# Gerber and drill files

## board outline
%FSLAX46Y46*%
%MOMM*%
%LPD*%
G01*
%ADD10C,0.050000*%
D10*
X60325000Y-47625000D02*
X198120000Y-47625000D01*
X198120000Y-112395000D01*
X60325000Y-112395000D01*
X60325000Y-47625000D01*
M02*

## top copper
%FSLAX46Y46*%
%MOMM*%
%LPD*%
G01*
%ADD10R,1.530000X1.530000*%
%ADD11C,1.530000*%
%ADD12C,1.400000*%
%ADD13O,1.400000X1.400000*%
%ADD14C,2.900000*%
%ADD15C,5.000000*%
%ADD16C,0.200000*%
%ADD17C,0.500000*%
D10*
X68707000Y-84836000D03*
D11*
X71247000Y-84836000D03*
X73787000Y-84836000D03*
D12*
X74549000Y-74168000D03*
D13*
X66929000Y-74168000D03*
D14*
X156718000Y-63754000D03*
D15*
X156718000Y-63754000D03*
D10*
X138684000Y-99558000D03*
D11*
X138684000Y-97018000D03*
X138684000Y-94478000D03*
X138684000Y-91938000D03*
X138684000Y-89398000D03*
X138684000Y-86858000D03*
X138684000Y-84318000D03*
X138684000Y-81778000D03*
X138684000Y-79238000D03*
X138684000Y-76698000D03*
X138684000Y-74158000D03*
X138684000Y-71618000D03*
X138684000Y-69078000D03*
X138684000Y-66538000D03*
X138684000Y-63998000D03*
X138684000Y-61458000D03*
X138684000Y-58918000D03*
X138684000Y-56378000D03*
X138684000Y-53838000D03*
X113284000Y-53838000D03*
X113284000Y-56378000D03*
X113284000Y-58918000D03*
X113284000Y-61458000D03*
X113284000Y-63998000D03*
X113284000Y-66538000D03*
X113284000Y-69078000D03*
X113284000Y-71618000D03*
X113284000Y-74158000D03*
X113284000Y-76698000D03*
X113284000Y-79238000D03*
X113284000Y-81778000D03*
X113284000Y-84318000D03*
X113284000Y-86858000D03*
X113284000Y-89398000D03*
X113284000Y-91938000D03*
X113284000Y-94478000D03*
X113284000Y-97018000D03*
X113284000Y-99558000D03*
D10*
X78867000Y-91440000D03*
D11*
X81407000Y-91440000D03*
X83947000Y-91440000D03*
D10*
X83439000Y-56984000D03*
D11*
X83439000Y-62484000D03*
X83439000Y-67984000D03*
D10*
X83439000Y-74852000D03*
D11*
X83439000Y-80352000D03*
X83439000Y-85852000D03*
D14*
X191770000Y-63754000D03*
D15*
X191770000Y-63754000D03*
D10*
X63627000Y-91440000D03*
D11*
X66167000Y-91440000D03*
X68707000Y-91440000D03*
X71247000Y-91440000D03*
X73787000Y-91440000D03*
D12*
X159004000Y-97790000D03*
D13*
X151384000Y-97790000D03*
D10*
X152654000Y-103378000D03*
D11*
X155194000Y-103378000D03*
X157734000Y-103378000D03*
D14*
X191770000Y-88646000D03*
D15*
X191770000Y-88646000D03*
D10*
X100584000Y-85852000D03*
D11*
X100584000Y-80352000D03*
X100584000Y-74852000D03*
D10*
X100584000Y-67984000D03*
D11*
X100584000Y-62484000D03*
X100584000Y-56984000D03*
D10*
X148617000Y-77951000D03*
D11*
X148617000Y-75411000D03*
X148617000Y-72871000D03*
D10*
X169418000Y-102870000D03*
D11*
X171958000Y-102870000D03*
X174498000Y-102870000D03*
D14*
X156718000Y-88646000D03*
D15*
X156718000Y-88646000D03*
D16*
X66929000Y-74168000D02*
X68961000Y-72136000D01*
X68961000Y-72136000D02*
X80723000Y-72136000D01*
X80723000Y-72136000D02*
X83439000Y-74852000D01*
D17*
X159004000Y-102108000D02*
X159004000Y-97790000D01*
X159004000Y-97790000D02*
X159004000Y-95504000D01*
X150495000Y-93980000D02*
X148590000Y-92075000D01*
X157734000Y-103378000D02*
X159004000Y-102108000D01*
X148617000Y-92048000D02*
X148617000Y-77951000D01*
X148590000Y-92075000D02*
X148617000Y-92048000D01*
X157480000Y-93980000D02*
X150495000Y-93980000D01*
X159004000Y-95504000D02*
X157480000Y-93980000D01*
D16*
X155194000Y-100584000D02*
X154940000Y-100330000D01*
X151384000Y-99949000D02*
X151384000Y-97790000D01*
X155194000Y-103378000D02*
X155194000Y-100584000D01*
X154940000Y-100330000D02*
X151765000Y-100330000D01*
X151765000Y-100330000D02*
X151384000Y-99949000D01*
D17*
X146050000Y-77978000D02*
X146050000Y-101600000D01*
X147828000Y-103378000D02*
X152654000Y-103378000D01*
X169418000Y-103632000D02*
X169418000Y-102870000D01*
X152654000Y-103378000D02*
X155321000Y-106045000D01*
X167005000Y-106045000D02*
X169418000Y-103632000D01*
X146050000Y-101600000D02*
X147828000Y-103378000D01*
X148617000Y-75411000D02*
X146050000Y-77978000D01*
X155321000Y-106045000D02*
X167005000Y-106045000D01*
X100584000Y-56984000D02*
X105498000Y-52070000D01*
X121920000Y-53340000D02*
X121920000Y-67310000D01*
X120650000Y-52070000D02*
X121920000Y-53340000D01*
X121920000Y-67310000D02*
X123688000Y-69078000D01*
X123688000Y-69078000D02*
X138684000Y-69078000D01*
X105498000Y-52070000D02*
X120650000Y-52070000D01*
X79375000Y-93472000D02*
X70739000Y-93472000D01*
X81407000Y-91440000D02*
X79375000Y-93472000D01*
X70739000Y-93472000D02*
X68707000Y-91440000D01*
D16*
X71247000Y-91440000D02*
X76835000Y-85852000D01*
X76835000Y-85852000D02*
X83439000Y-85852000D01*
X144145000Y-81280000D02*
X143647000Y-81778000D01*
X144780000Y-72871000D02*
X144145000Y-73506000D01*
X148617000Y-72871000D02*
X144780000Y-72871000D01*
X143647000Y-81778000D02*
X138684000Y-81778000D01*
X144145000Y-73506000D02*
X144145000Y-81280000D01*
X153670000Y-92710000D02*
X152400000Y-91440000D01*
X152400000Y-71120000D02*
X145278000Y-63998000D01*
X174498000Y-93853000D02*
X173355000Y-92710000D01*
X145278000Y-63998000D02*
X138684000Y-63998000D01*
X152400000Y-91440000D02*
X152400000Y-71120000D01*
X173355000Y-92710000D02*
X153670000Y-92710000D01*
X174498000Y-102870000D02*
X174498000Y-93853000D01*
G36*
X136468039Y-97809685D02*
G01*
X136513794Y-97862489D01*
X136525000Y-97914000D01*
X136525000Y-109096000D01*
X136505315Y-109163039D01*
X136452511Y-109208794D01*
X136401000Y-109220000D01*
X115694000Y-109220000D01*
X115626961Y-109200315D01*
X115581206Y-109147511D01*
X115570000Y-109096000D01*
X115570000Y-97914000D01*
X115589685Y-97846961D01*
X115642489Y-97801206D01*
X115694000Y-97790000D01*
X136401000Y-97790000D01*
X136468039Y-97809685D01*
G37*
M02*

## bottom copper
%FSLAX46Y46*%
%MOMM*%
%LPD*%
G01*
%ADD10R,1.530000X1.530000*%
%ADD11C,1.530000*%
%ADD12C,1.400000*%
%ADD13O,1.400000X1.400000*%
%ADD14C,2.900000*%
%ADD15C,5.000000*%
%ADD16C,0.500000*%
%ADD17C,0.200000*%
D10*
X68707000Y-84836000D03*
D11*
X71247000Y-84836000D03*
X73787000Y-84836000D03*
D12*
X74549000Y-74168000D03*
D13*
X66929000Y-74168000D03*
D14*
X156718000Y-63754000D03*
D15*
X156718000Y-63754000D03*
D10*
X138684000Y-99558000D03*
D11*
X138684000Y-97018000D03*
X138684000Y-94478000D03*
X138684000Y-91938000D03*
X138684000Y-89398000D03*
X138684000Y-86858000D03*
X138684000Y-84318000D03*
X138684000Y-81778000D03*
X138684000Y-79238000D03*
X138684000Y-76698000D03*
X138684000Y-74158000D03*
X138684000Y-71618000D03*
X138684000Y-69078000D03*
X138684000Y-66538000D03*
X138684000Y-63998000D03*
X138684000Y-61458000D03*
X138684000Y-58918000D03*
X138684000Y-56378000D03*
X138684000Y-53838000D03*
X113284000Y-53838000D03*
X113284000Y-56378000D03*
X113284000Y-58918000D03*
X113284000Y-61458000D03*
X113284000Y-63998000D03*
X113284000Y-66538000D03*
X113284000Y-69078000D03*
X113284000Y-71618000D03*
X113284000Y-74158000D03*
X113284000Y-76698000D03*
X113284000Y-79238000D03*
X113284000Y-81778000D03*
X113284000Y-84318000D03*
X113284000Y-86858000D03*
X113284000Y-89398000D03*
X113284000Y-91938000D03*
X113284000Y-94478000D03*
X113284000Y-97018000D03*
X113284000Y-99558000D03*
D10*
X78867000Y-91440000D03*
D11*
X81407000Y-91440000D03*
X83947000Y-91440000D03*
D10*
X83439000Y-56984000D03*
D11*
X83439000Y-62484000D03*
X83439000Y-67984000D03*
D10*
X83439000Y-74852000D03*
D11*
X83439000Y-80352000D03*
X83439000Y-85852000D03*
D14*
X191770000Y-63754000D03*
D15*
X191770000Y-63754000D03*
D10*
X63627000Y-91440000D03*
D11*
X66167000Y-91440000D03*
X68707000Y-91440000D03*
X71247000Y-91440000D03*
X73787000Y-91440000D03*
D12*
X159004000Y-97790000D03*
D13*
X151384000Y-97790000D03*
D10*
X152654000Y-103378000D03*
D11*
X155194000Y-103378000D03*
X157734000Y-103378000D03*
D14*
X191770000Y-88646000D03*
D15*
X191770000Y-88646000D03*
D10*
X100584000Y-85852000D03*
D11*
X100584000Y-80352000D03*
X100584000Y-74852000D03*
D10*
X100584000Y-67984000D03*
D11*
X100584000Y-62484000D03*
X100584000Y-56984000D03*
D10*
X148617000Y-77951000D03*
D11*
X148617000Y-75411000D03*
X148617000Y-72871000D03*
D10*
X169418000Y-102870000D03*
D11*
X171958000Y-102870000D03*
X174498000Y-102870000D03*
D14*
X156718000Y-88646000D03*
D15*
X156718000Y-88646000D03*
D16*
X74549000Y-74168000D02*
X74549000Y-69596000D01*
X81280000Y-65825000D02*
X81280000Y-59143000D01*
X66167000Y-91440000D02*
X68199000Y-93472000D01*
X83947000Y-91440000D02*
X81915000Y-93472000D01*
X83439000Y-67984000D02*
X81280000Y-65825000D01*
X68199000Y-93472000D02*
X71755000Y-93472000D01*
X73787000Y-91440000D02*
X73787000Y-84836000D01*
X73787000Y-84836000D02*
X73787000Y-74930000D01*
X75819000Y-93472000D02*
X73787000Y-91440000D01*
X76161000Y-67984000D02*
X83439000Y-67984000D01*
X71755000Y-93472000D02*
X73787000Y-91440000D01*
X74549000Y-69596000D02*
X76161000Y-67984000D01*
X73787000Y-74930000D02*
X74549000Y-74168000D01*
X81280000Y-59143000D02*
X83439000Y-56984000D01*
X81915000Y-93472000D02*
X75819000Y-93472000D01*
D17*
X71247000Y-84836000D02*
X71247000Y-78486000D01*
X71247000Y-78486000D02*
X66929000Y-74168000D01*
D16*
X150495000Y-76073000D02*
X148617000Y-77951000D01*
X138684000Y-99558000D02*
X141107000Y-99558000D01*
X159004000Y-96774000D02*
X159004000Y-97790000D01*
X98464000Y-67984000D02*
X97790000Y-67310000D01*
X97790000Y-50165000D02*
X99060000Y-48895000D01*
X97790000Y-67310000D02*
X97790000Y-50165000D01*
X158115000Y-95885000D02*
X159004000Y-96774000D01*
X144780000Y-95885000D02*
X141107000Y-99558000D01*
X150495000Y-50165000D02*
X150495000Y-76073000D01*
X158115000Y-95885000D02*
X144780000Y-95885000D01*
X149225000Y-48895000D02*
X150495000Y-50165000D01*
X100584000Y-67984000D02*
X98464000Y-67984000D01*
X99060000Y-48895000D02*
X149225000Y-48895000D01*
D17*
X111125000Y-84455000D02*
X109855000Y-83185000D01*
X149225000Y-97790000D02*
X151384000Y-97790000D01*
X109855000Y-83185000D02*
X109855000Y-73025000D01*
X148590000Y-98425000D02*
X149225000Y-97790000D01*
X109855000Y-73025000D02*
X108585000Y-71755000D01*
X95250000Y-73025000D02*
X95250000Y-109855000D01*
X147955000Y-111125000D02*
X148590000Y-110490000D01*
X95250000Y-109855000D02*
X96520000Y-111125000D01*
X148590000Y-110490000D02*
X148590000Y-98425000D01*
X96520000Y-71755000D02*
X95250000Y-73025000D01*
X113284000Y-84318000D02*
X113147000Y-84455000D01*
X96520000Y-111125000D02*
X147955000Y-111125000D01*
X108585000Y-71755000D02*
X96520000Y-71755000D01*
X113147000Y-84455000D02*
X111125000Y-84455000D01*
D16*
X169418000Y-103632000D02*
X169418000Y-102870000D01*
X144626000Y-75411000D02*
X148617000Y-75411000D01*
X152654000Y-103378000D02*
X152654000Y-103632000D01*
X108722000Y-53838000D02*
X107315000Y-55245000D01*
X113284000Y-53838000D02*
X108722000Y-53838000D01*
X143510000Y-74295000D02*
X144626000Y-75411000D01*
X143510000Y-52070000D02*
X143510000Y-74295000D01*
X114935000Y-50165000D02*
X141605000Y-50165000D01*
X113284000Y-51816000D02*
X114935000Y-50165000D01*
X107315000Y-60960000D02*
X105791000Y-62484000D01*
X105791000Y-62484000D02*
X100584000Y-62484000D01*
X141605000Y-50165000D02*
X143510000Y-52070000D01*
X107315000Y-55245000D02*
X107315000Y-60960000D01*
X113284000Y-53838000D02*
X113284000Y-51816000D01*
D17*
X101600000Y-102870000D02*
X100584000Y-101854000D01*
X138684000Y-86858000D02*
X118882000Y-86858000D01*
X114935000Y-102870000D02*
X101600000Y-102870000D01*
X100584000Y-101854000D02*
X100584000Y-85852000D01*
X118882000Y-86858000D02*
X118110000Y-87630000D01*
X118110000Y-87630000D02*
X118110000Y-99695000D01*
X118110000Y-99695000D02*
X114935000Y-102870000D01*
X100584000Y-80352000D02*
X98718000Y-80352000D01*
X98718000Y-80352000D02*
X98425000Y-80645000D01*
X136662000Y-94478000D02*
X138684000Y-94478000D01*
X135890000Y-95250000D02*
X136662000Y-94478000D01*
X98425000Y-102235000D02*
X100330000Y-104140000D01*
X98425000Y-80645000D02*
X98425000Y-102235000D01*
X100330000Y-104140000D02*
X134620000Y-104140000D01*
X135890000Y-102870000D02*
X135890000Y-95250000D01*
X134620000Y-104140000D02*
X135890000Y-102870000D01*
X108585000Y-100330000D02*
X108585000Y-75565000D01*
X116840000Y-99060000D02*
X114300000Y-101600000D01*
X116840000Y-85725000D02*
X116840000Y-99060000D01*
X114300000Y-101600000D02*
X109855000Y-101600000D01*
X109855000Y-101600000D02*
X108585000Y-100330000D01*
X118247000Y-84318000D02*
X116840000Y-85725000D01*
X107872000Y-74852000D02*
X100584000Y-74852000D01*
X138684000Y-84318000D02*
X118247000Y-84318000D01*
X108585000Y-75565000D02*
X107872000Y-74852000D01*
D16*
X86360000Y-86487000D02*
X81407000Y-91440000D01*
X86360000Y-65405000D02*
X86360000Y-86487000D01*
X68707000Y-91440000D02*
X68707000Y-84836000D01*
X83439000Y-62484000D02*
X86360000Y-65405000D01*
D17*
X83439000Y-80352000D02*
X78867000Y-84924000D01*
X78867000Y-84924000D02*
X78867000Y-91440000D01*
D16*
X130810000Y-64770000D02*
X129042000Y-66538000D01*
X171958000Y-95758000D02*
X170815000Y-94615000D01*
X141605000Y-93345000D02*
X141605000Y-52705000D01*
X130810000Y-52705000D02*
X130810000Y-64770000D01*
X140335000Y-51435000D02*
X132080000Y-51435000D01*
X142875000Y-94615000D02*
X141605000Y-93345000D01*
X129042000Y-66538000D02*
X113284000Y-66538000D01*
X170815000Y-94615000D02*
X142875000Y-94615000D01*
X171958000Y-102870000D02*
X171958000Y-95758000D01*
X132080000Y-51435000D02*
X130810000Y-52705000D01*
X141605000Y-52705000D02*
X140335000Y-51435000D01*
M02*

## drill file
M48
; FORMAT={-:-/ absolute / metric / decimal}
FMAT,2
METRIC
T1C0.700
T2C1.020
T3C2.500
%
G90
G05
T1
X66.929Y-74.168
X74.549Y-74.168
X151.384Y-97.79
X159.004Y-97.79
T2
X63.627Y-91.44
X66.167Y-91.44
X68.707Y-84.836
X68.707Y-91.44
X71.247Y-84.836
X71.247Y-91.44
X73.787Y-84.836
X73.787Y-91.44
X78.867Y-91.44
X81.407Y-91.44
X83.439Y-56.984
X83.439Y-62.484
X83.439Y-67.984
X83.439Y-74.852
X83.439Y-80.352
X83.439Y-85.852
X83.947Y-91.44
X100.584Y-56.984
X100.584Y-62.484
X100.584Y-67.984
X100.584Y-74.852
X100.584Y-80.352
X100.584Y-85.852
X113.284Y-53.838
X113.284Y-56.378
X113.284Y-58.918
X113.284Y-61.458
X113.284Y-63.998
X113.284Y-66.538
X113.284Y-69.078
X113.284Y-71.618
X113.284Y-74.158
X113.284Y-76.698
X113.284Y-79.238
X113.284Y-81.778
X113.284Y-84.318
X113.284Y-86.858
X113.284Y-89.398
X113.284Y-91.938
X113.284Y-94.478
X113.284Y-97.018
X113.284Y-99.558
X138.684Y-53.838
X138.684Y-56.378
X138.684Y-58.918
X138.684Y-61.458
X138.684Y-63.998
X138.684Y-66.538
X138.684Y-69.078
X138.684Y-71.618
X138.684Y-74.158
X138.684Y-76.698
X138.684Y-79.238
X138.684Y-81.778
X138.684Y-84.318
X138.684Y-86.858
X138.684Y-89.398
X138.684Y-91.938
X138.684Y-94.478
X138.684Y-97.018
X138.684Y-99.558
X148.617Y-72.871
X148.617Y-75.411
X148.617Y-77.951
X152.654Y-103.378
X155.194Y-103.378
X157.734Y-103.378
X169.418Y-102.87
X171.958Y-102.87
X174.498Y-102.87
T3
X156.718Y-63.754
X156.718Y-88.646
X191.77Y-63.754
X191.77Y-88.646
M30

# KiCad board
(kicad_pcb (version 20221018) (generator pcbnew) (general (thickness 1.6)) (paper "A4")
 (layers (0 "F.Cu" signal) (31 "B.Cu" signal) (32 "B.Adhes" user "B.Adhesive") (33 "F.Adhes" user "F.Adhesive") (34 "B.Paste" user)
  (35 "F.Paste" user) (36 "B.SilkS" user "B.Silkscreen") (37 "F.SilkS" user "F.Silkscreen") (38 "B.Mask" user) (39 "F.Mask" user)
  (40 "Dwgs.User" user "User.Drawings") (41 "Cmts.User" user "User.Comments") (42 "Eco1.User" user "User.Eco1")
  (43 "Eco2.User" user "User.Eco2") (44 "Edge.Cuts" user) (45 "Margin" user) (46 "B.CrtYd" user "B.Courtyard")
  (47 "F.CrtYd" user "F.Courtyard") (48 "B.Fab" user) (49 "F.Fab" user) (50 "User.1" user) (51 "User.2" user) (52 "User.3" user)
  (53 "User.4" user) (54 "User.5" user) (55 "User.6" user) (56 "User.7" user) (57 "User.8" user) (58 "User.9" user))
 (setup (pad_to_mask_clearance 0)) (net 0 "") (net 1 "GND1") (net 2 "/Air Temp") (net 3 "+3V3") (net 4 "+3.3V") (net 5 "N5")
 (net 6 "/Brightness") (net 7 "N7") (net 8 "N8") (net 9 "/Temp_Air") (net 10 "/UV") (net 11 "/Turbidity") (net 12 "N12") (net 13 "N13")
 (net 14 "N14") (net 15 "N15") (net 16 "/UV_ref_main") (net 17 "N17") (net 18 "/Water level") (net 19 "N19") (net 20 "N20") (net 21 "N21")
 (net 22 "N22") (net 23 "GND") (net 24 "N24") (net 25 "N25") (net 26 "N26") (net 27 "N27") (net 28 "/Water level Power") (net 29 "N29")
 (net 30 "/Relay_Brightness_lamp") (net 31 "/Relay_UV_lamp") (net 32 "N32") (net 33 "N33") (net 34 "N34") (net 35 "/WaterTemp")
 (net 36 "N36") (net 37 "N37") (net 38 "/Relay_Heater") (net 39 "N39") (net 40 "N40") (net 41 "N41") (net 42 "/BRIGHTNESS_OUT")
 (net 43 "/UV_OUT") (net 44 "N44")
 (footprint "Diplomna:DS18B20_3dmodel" (layer "F.Cu") (at 76.327 87.376)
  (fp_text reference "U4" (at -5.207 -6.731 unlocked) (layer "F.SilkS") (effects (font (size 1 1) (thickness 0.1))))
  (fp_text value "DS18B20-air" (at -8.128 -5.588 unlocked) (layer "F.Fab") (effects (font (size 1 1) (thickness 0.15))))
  (pad "1" thru_hole rect (at -7.62 -2.54) (size 1.53 1.53) (drill 1.02) (layers "*.Cu" "*.Mask") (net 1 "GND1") (solder_mask_margin 0.102))
  (pad "2" thru_hole circle (at -5.08 -2.54) (size 1.53 1.53) (drill 1.02) (layers "*.Cu" "*.Mask") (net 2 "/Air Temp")
   (solder_mask_margin 0.102))
  (pad "3" thru_hole circle (at -2.54 -2.54) (size 1.53 1.53) (drill 1.02) (layers "*.Cu" "*.Mask") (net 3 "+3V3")
   (solder_mask_margin 0.102)))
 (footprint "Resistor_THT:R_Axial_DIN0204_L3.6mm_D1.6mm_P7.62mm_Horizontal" (layer "F.Cu") (at 74.549 74.168 180)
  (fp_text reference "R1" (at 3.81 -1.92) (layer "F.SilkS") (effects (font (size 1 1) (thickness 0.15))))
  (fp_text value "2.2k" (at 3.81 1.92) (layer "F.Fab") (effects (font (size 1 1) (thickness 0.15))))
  (pad "1" thru_hole circle (at 0 0 180) (size 1.4 1.4) (drill 0.7) (layers "*.Cu" "*.Mask") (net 3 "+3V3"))
  (pad "2" thru_hole oval (at 7.62 0 180) (size 1.4 1.4) (drill 0.7) (layers "*.Cu" "*.Mask") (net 2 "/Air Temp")))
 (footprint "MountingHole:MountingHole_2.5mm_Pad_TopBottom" (layer "F.Cu") (at 156.718 63.754)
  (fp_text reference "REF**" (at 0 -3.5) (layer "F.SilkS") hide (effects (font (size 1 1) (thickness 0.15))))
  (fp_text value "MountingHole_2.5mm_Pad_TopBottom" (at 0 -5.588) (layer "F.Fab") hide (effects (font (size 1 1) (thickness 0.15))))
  (pad "1" thru_hole circle (at 0 0) (size 2.9 2.9) (drill 2.5) (layers "*.Cu" "*.Mask"))
  (pad "1" connect circle (at 0 0) (size 5 5) (layers "F.Cu" "F.Mask"))
  (pad "1" connect circle (at 0 0) (size 5 5) (layers "B.Cu" "B.Mask")))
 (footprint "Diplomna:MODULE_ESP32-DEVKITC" (layer "F.Cu") (at 125.984 76.708 180)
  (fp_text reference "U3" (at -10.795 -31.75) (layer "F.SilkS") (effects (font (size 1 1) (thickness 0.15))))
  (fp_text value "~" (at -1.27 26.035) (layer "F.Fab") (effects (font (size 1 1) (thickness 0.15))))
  (pad "1" thru_hole rect (at -12.7 -22.85 180) (size 1.53 1.53) (drill 1.02) (layers "*.Cu" "*.Mask") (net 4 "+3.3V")
   (solder_mask_margin 0.102))
  (pad "2" thru_hole circle (at -12.7 -20.31 180) (size 1.53 1.53) (drill 1.02) (layers "*.Cu" "*.Mask") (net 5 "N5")
   (solder_mask_margin 0.102))
  (pad "3" thru_hole circle (at -12.7 -17.77 180) (size 1.53 1.53) (drill 1.02) (layers "*.Cu" "*.Mask") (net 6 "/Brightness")
   (solder_mask_margin 0.102))
  (pad "4" thru_hole circle (at -12.7 -15.23 180) (size 1.53 1.53) (drill 1.02) (layers "*.Cu" "*.Mask") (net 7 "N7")
   (solder_mask_margin 0.102))
  (pad "5" thru_hole circle (at -12.7 -12.69 180) (size 1.53 1.53) (drill 1.02) (layers "*.Cu" "*.Mask") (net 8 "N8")
   (solder_mask_margin 0.102))
  (pad "6" thru_hole circle (at -12.7 -10.15 180) (size 1.53 1.53) (drill 1.02) (layers "*.Cu" "*.Mask") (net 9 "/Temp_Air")
   (solder_mask_margin 0.102))
  (pad "7" thru_hole circle (at -12.7 -7.61 180) (size 1.53 1.53) (drill 1.02) (layers "*.Cu" "*.Mask") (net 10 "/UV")
   (solder_mask_margin 0.102))
  (pad "8" thru_hole circle (at -12.7 -5.07 180) (size 1.53 1.53) (drill 1.02) (layers "*.Cu" "*.Mask") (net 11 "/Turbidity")
   (solder_mask_margin 0.102))
  (pad "9" thru_hole circle (at -12.7 -2.53 180) (size 1.53 1.53) (drill 1.02) (layers "*.Cu" "*.Mask") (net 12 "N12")
   (solder_mask_margin 0.102))
  (pad "10" thru_hole circle (at -12.7 0.01 180) (size 1.53 1.53) (drill 1.02) (layers "*.Cu" "*.Mask") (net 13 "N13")
   (solder_mask_margin 0.102))
  (pad "11" thru_hole circle (at -12.7 2.55 180) (size 1.53 1.53) (drill 1.02) (layers "*.Cu" "*.Mask") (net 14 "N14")
   (solder_mask_margin 0.102))
  (pad "12" thru_hole circle (at -12.7 5.09 180) (size 1.53 1.53) (drill 1.02) (layers "*.Cu" "*.Mask") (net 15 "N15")
   (solder_mask_margin 0.102))
  (pad "13" thru_hole circle (at -12.7 7.63 180) (size 1.53 1.53) (drill 1.02) (layers "*.Cu" "*.Mask") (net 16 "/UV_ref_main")
   (solder_mask_margin 0.102))
  (pad "14" thru_hole circle (at -12.7 10.17 180) (size 1.53 1.53) (drill 1.02) (layers "*.Cu" "*.Mask") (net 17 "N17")
   (solder_mask_margin 0.102))
  (pad "15" thru_hole circle (at -12.7 12.71 180) (size 1.53 1.53) (drill 1.02) (layers "*.Cu" "*.Mask") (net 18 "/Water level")
   (solder_mask_margin 0.102))
  (pad "16" thru_hole circle (at -12.7 15.25 180) (size 1.53 1.53) (drill 1.02) (layers "*.Cu" "*.Mask") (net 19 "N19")
   (solder_mask_margin 0.102))
  (pad "17" thru_hole circle (at -12.7 17.79 180) (size 1.53 1.53) (drill 1.02) (layers "*.Cu" "*.Mask") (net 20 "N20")
   (solder_mask_margin 0.102))
  (pad "18" thru_hole circle (at -12.7 20.33 180) (size 1.53 1.53) (drill 1.02) (layers "*.Cu" "*.Mask") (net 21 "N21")
   (solder_mask_margin 0.102))
  (pad "19" thru_hole circle (at -12.7 22.87 180) (size 1.53 1.53) (drill 1.02) (layers "*.Cu" "*.Mask") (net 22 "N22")
   (solder_mask_margin 0.102))
  (pad "20" thru_hole circle (at 12.7 22.87 180) (size 1.53 1.53) (drill 1.02) (layers "*.Cu" "*.Mask") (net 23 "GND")
   (solder_mask_margin 0.102))
  (pad "21" thru_hole circle (at 12.7 20.33 180) (size 1.53 1.53) (drill 1.02) (layers "*.Cu" "*.Mask") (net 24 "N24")
   (solder_mask_margin 0.102))
  (pad "22" thru_hole circle (at 12.7 17.79 180) (size 1.53 1.53) (drill 1.02) (layers "*.Cu" "*.Mask") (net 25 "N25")
   (solder_mask_margin 0.102))
  (pad "23" thru_hole circle (at 12.7 15.25 180) (size 1.53 1.53) (drill 1.02) (layers "*.Cu" "*.Mask") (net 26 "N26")
   (solder_mask_margin 0.102))
  (pad "24" thru_hole circle (at 12.7 12.71 180) (size 1.53 1.53) (drill 1.02) (layers "*.Cu" "*.Mask") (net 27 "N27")
   (solder_mask_margin 0.102))
  (pad "25" thru_hole circle (at 12.7 10.17 180) (size 1.53 1.53) (drill 1.02) (layers "*.Cu" "*.Mask") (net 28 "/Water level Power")
   (solder_mask_margin 0.102))
  (pad "26" thru_hole circle (at 12.7 7.63 180) (size 1.53 1.53) (drill 1.02) (layers "*.Cu" "*.Mask") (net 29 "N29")
   (solder_mask_margin 0.102))
  (pad "27" thru_hole circle (at 12.7 5.09 180) (size 1.53 1.53) (drill 1.02) (layers "*.Cu" "*.Mask") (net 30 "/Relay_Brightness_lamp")
   (solder_mask_margin 0.102))
  (pad "28" thru_hole circle (at 12.7 2.55 180) (size 1.53 1.53) (drill 1.02) (layers "*.Cu" "*.Mask") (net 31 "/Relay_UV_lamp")
   (solder_mask_margin 0.102))
  (pad "29" thru_hole circle (at 12.7 0.01 180) (size 1.53 1.53) (drill 1.02) (layers "*.Cu" "*.Mask") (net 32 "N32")
   (solder_mask_margin 0.102))
  (pad "30" thru_hole circle (at 12.7 -2.53 180) (size 1.53 1.53) (drill 1.02) (layers "*.Cu" "*.Mask") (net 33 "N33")
   (solder_mask_margin 0.102))
  (pad "31" thru_hole circle (at 12.7 -5.07 180) (size 1.53 1.53) (drill 1.02) (layers "*.Cu" "*.Mask") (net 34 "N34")
   (solder_mask_margin 0.102))
  (pad "32" thru_hole circle (at 12.7 -7.61 180) (size 1.53 1.53) (drill 1.02) (layers "*.Cu" "*.Mask") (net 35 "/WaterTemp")
   (solder_mask_margin 0.102))
  (pad "33" thru_hole circle (at 12.7 -10.15 180) (size 1.53 1.53) (drill 1.02) (layers "*.Cu" "*.Mask") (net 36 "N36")
   (solder_mask_margin 0.102))
  (pad "34" thru_hole circle (at 12.7 -12.69 180) (size 1.53 1.53) (drill 1.02) (layers "*.Cu" "*.Mask") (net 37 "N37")
   (solder_mask_margin 0.102))
  (pad "35" thru_hole circle (at 12.7 -15.23 180) (size 1.53 1.53) (drill 1.02) (layers "*.Cu" "*.Mask") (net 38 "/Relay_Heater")
   (solder_mask_margin 0.102))
  (pad "36" thru_hole circle (at 12.7 -17.77 180) (size 1.53 1.53) (drill 1.02) (layers "*.Cu" "*.Mask") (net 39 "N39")
   (solder_mask_margin 0.102))
  (pad "37" thru_hole circle (at 12.7 -20.31 180) (size 1.53 1.53) (drill 1.02) (layers "*.Cu" "*.Mask") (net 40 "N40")
   (solder_mask_margin 0.102))
  (pad "38" thru_hole circle (at 12.7 -22.85 180) (size 1.53 1.53) (drill 1.02) (layers "*.Cu" "*.Mask") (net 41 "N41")
   (solder_mask_margin 0.102)))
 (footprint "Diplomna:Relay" (layer "F.Cu") (at 254.508 101.092 -90)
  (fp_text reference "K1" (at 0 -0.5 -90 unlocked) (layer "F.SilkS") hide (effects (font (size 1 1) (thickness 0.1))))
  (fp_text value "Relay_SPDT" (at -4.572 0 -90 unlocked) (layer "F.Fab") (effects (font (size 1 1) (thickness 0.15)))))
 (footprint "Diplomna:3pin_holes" (layer "F.Cu") (at 86.487 93.98)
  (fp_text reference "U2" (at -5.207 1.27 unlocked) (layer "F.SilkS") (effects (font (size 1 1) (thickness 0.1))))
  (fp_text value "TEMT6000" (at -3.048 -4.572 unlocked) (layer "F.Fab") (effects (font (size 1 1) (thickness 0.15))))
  (pad "1" thru_hole rect (at -7.62 -2.54) (size 1.53 1.53) (drill 1.02) (layers "*.Cu" "*.Mask") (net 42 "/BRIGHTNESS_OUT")
   (solder_mask_margin 0.102))
  (pad "2" thru_hole circle (at -5.08 -2.54) (size 1.53 1.53) (drill 1.02) (layers "*.Cu" "*.Mask") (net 1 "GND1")
   (solder_mask_margin 0.102))
  (pad "3" thru_hole circle (at -2.54 -2.54) (size 1.53 1.53) (drill 1.02) (layers "*.Cu" "*.Mask") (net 3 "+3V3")
   (solder_mask_margin 0.102)))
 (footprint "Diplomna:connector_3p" (layer "F.Cu") (at 83.439 62.484 -90)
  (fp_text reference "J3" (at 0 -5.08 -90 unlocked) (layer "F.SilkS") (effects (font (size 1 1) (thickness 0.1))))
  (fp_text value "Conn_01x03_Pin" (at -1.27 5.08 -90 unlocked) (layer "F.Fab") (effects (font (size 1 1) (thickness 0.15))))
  (pad "1" thru_hole rect (at -5.5 0 270) (size 1.53 1.53) (drill 1.02) (layers "*.Cu" "*.Mask") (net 3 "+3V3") (solder_mask_margin 0.102))
  (pad "2" thru_hole circle (at 0 0 270) (size 1.53 1.53) (drill 1.02) (layers "*.Cu" "*.Mask") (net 1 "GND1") (solder_mask_margin 0.102))
  (pad "3" thru_hole circle (at 5.5 0 270) (size 1.53 1.53) (drill 1.02) (layers "*.Cu" "*.Mask") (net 3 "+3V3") (solder_mask_margin 0.102)))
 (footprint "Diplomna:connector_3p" (layer "F.Cu") (at 83.439 80.352 -90)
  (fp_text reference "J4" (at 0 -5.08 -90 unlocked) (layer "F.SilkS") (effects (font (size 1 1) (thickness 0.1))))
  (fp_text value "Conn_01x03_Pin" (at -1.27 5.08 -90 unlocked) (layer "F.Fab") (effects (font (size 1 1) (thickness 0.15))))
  (pad "1" thru_hole rect (at -5.5 0 270) (size 1.53 1.53) (drill 1.02) (layers "*.Cu" "*.Mask") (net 2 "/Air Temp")
   (solder_mask_margin 0.102))
  (pad "2" thru_hole circle (at 0 0 270) (size 1.53 1.53) (drill 1.02) (layers "*.Cu" "*.Mask") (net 42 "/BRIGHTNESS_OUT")
   (solder_mask_margin 0.102))
  (pad "3" thru_hole circle (at 5.5 0 270) (size 1.53 1.53) (drill 1.02) (layers "*.Cu" "*.Mask") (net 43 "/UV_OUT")
   (solder_mask_margin 0.102)))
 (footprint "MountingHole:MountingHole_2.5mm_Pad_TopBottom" (layer "F.Cu") (at 191.77 63.754)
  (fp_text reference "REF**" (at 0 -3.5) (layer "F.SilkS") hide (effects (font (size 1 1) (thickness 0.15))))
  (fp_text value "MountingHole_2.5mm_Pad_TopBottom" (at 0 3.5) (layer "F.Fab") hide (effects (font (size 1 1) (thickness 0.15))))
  (pad "1" thru_hole circle (at 0 0) (size 2.9 2.9) (drill 2.5) (layers "*.Cu" "*.Mask"))
  (pad "1" connect circle (at 0 0) (size 5 5) (layers "F.Cu" "F.Mask"))
  (pad "1" connect circle (at 0 0) (size 5 5) (layers "B.Cu" "B.Mask")))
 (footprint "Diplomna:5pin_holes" (layer "F.Cu") (at 78.867 97.155)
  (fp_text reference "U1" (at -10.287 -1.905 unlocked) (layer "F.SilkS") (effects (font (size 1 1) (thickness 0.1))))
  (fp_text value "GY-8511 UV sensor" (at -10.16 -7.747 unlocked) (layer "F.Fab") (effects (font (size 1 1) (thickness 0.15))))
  (pad "1" thru_hole rect (at -15.24 -5.715) (size 1.53 1.53) (drill 1.02) (layers "*.Cu" "*.Mask") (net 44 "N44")
   (solder_mask_margin 0.102))
  (pad "2" thru_hole circle (at -12.7 -5.715) (size 1.53 1.53) (drill 1.02) (layers "*.Cu" "*.Mask") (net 3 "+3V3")
   (solder_mask_margin 0.102))
  (pad "3" thru_hole circle (at -10.16 -5.715) (size 1.53 1.53) (drill 1.02) (layers "*.Cu" "*.Mask") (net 1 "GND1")
   (solder_mask_margin 0.102))
  (pad "4" thru_hole circle (at -7.62 -5.715) (size 1.53 1.53) (drill 1.02) (layers "*.Cu" "*.Mask") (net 43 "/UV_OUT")
   (solder_mask_margin 0.102))
  (pad "5" thru_hole circle (at -5.08 -5.715) (size 1.53 1.53) (drill 1.02) (layers "*.Cu" "*.Mask") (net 3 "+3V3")
   (solder_mask_margin 0.102)))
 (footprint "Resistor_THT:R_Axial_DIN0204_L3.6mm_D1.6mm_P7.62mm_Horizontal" (layer "F.Cu") (at 159.004 97.79 180)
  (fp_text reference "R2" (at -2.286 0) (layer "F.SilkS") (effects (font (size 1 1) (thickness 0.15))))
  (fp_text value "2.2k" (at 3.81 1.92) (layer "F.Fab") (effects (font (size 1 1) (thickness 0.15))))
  (pad "1" thru_hole circle (at 0 0 180) (size 1.4 1.4) (drill 0.7) (layers "*.Cu" "*.Mask") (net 4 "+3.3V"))
  (pad "2" thru_hole oval (at 7.62 0 180) (size 1.4 1.4) (drill 0.7) (layers "*.Cu" "*.Mask") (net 35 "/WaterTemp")))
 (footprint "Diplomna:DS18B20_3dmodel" (layer "F.Cu") (at 160.274 105.918)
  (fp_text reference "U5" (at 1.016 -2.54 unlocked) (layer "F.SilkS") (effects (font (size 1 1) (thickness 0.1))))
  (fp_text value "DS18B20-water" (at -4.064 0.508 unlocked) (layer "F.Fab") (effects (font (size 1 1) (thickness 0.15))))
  (pad "1" thru_hole rect (at -7.62 -2.54) (size 1.53 1.53) (drill 1.02) (layers "*.Cu" "*.Mask") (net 23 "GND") (solder_mask_margin 0.102))
  (pad "2" thru_hole circle (at -5.08 -2.54) (size 1.53 1.53) (drill 1.02) (layers "*.Cu" "*.Mask") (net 35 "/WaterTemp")
   (solder_mask_margin 0.102))
  (pad "3" thru_hole circle (at -2.54 -2.54) (size 1.53 1.53) (drill 1.02) (layers "*.Cu" "*.Mask") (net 4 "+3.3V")
   (solder_mask_margin 0.102)))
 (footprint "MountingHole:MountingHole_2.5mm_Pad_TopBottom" (layer "F.Cu") (at 191.77 88.646)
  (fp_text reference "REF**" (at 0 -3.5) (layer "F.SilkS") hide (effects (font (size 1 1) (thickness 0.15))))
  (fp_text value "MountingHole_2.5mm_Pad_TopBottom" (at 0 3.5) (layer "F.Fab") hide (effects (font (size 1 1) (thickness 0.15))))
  (pad "1" thru_hole circle (at 0 0) (size 2.9 2.9) (drill 2.5) (layers "*.Cu" "*.Mask"))
  (pad "1" connect circle (at 0 0) (size 5 5) (layers "F.Cu" "F.Mask"))
  (pad "1" connect circle (at 0 0) (size 5 5) (layers "B.Cu" "B.Mask")))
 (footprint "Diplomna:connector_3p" (layer "F.Cu") (at 100.584 80.352 90)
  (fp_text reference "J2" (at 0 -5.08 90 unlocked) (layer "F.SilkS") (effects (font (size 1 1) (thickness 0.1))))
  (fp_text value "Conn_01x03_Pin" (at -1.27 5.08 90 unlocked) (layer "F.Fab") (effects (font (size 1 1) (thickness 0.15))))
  (pad "1" thru_hole rect (at -5.5 0 90) (size 1.53 1.53) (drill 1.02) (layers "*.Cu" "*.Mask") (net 9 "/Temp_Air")
   (solder_mask_margin 0.102))
  (pad "2" thru_hole circle (at 0 0 90) (size 1.53 1.53) (drill 1.02) (layers "*.Cu" "*.Mask") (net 6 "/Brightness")
   (solder_mask_margin 0.102))
  (pad "3" thru_hole circle (at 5.5 0 90) (size 1.53 1.53) (drill 1.02) (layers "*.Cu" "*.Mask") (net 10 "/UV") (solder_mask_margin 0.102)))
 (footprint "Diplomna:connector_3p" (layer "F.Cu") (at 100.584 62.484 90)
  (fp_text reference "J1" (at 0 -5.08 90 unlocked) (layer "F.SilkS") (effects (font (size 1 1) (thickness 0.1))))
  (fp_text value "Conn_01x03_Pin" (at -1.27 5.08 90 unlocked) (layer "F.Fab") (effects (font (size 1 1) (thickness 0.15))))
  (pad "1" thru_hole rect (at -5.5 0 90) (size 1.53 1.53) (drill 1.02) (layers "*.Cu" "*.Mask") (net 4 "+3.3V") (solder_mask_margin 0.102))
  (pad "2" thru_hole circle (at 0 0 90) (size 1.53 1.53) (drill 1.02) (layers "*.Cu" "*.Mask") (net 23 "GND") (solder_mask_margin 0.102))
  (pad "3" thru_hole circle (at 5.5 0 90) (size 1.53 1.53) (drill 1.02) (layers "*.Cu" "*.Mask") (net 16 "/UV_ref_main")
   (solder_mask_margin 0.102)))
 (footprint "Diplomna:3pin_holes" (layer "F.Cu") (at 151.157 70.331 90)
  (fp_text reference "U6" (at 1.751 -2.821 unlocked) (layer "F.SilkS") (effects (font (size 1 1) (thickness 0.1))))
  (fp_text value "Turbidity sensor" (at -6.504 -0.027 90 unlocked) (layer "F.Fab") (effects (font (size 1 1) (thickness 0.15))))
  (pad "1" thru_hole rect (at -7.62 -2.54 90) (size 1.53 1.53) (drill 1.02) (layers "*.Cu" "*.Mask") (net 4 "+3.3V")
   (solder_mask_margin 0.102))
  (pad "2" thru_hole circle (at -5.08 -2.54 90) (size 1.53 1.53) (drill 1.02) (layers "*.Cu" "*.Mask") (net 23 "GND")
   (solder_mask_margin 0.102))
  (pad "3" thru_hole circle (at -2.54 -2.54 90) (size 1.53 1.53) (drill 1.02) (layers "*.Cu" "*.Mask") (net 11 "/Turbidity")
   (solder_mask_margin 0.102)))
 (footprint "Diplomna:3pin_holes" (layer "F.Cu") (at 177.038 105.41)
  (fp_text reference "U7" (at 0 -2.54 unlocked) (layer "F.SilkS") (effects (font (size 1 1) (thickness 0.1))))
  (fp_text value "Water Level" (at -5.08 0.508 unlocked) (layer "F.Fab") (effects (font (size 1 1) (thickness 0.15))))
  (pad "1" thru_hole rect (at -7.62 -2.54) (size 1.53 1.53) (drill 1.02) (layers "*.Cu" "*.Mask") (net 23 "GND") (solder_mask_margin 0.102))
  (pad "2" thru_hole circle (at -5.08 -2.54) (size 1.53 1.53) (drill 1.02) (layers "*.Cu" "*.Mask") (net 28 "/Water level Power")
   (solder_mask_margin 0.102))
  (pad "3" thru_hole circle (at -2.54 -2.54) (size 1.53 1.53) (drill 1.02) (layers "*.Cu" "*.Mask") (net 18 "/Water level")
   (solder_mask_margin 0.102)))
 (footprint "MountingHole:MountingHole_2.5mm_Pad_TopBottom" (layer "F.Cu") (at 156.718 88.646)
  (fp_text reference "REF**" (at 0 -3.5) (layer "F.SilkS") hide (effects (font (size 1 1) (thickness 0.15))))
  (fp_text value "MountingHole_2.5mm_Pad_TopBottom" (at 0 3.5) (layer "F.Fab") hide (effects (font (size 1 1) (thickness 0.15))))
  (pad "1" thru_hole circle (at 0 0) (size 2.9 2.9) (drill 2.5) (layers "*.Cu" "*.Mask"))
  (pad "1" connect circle (at 0 0) (size 5 5) (layers "F.Cu" "F.Mask"))
  (pad "1" connect circle (at 0 0) (size 5 5) (layers "B.Cu" "B.Mask")))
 (gr_rect (start 60.325 47.625) (end 198.12 112.395) (stroke (width 0.05) (type default)) (fill none) (layer "Edge.Cuts"))
 (segment (start 74.549 74.168) (end 74.549 69.596) (width 0.5) (layer "B.Cu") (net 3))
 (segment (start 81.28 65.825) (end 81.28 59.143) (width 0.5) (layer "B.Cu") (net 3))
 (segment (start 66.167 91.44) (end 68.199 93.472) (width 0.5) (layer "B.Cu") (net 3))
 (segment (start 83.947 91.44) (end 81.915 93.472) (width 0.5) (layer "B.Cu") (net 3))
 (segment (start 83.439 67.984) (end 81.28 65.825) (width 0.5) (layer "B.Cu") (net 3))
 (segment (start 68.199 93.472) (end 71.755 93.472) (width 0.5) (layer "B.Cu") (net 3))
 (segment (start 73.787 91.44) (end 73.787 84.836) (width 0.5) (layer "B.Cu") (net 3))
 (segment (start 73.787 84.836) (end 73.787 74.93) (width 0.5) (layer "B.Cu") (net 3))
 (segment (start 75.819 93.472) (end 73.787 91.44) (width 0.5) (layer "B.Cu") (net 3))
 (segment (start 76.161 67.984) (end 83.439 67.984) (width 0.5) (layer "B.Cu") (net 3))
 (segment (start 71.755 93.472) (end 73.787 91.44) (width 0.5) (layer "B.Cu") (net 3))
 (segment (start 74.549 69.596) (end 76.161 67.984) (width 0.5) (layer "B.Cu") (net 3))
 (segment (start 73.787 74.93) (end 74.549 74.168) (width 0.5) (layer "B.Cu") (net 3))
 (segment (start 81.28 59.143) (end 83.439 56.984) (width 0.5) (layer "B.Cu") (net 3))
 (segment (start 81.915 93.472) (end 75.819 93.472) (width 0.5) (layer "B.Cu") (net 3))
 (segment (start 66.929 74.168) (end 68.961 72.136) (width 0.2) (layer "F.Cu") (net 2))
 (segment (start 68.961 72.136) (end 80.723 72.136) (width 0.2) (layer "F.Cu") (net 2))
 (segment (start 80.723 72.136) (end 83.439 74.852) (width 0.2) (layer "F.Cu") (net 2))
 (segment (start 71.247 84.836) (end 71.247 78.486) (width 0.2) (layer "B.Cu") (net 2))
 (segment (start 71.247 78.486) (end 66.929 74.168) (width 0.2) (layer "B.Cu") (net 2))
 (segment (start 159.004 102.108) (end 159.004 97.79) (width 0.5) (layer "F.Cu") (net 4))
 (segment (start 159.004 97.79) (end 159.004 95.504) (width 0.5) (layer "F.Cu") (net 4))
 (segment (start 150.495 93.98) (end 148.59 92.075) (width 0.5) (layer "F.Cu") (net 4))
 (segment (start 157.734 103.378) (end 159.004 102.108) (width 0.5) (layer "F.Cu") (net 4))
 (segment (start 148.617 92.048) (end 148.617 77.951) (width 0.5) (layer "F.Cu") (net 4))
 (segment (start 148.59 92.075) (end 148.617 92.048) (width 0.5) (layer "F.Cu") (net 4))
 (segment (start 157.48 93.98) (end 150.495 93.98) (width 0.5) (layer "F.Cu") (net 4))
 (segment (start 159.004 95.504) (end 157.48 93.98) (width 0.5) (layer "F.Cu") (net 4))
 (segment (start 150.495 76.073) (end 148.617 77.951) (width 0.5) (layer "B.Cu") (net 4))
 (segment (start 138.684 99.558) (end 141.107 99.558) (width 0.5) (layer "B.Cu") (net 4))
 (segment (start 159.004 96.774) (end 159.004 97.79) (width 0.5) (layer "B.Cu") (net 4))
 (segment (start 98.464 67.984) (end 97.79 67.31) (width 0.5) (layer "B.Cu") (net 4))
 (segment (start 97.79 50.165) (end 99.06 48.895) (width 0.5) (layer "B.Cu") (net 4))
 (segment (start 97.79 67.31) (end 97.79 50.165) (width 0.5) (layer "B.Cu") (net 4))
 (segment (start 158.115 95.885) (end 159.004 96.774) (width 0.5) (layer "B.Cu") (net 4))
 (segment (start 144.78 95.885) (end 141.107 99.558) (width 0.5) (layer "B.Cu") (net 4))
 (segment (start 150.495 50.165) (end 150.495 76.073) (width 0.5) (layer "B.Cu") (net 4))
 (segment (start 158.115 95.885) (end 144.78 95.885) (width 0.5) (layer "B.Cu") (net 4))
 (segment (start 149.225 48.895) (end 150.495 50.165) (width 0.5) (layer "B.Cu") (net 4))
 (segment (start 100.584 67.984) (end 98.464 67.984) (width 0.5) (layer "B.Cu") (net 4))
 (segment (start 99.06 48.895) (end 149.225 48.895) (width 0.5) (layer "B.Cu") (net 4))
 (segment (start 155.194 100.584) (end 154.94 100.33) (width 0.2) (layer "F.Cu") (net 35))
 (segment (start 151.384 99.949) (end 151.384 97.79) (width 0.2) (layer "F.Cu") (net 35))
 (segment (start 155.194 103.378) (end 155.194 100.584) (width 0.2) (layer "F.Cu") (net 35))
 (segment (start 154.94 100.33) (end 151.765 100.33) (width 0.2) (layer "F.Cu") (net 35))
 (segment (start 151.765 100.33) (end 151.384 99.949) (width 0.2) (layer "F.Cu") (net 35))
 (segment (start 111.125 84.455) (end 109.855 83.185) (width 0.2) (layer "B.Cu") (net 35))
 (segment (start 149.225 97.79) (end 151.384 97.79) (width 0.2) (layer "B.Cu") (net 35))
 (segment (start 109.855 83.185) (end 109.855 73.025) (width 0.2) (layer "B.Cu") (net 35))
 (segment (start 148.59 98.425) (end 149.225 97.79) (width 0.2) (layer "B.Cu") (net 35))
 (segment (start 109.855 73.025) (end 108.585 71.755) (width 0.2) (layer "B.Cu") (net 35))
 (segment (start 95.25 73.025) (end 95.25 109.855) (width 0.2) (layer "B.Cu") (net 35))
 (segment (start 147.955 111.125) (end 148.59 110.49) (width 0.2) (layer "B.Cu") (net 35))
 (segment (start 95.25 109.855) (end 96.52 111.125) (width 0.2) (layer "B.Cu") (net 35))
 (segment (start 148.59 110.49) (end 148.59 98.425) (width 0.2) (layer "B.Cu") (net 35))
 (segment (start 96.52 71.755) (end 95.25 73.025) (width 0.2) (layer "B.Cu") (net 35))
 (segment (start 113.284 84.318) (end 113.147 84.455) (width 0.2) (layer "B.Cu") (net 35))
 (segment (start 96.52 111.125) (end 147.955 111.125) (width 0.2) (layer "B.Cu") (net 35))
 (segment (start 108.585 71.755) (end 96.52 71.755) (width 0.2) (layer "B.Cu") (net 35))
 (segment (start 113.147 84.455) (end 111.125 84.455) (width 0.2) (layer "B.Cu") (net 35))
 (segment (start 146.05 77.978) (end 146.05 101.6) (width 0.5) (layer "F.Cu") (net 23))
 (segment (start 147.828 103.378) (end 152.654 103.378) (width 0.5) (layer "F.Cu") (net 23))
 (segment (start 169.418 103.632) (end 169.418 102.87) (width 0.5) (layer "F.Cu") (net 23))
 (segment (start 152.654 103.378) (end 155.321 106.045) (width 0.5) (layer "F.Cu") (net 23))
 (segment (start 167.005 106.045) (end 169.418 103.632) (width 0.5) (layer "F.Cu") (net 23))
 (segment (start 146.05 101.6) (end 147.828 103.378) (width 0.5) (layer "F.Cu") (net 23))
 (segment (start 148.617 75.411) (end 146.05 77.978) (width 0.5) (layer "F.Cu") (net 23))
 (segment (start 155.321 106.045) (end 167.005 106.045) (width 0.5) (layer "F.Cu") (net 23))
 (segment (start 169.418 103.632) (end 169.418 102.87) (width 0.5) (layer "B.Cu") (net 23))
 (segment (start 144.626 75.411) (end 148.617 75.411) (width 0.5) (layer "B.Cu") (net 23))
 (segment (start 152.654 103.378) (end 152.654 103.632) (width 0.5) (layer "B.Cu") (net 23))
 (segment (start 108.722 53.838) (end 107.315 55.245) (width 0.5) (layer "B.Cu") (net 23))
 (segment (start 113.284 53.838) (end 108.722 53.838) (width 0.5) (layer "B.Cu") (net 23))
 (segment (start 143.51 74.295) (end 144.626 75.411) (width 0.5) (layer "B.Cu") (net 23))
 (segment (start 143.51 52.07) (end 143.51 74.295) (width 0.5) (layer "B.Cu") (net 23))
 (segment (start 114.935 50.165) (end 141.605 50.165) (width 0.5) (layer "B.Cu") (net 23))
 (segment (start 113.284 51.816) (end 114.935 50.165) (width 0.5) (layer "B.Cu") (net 23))
 (segment (start 107.315 60.96) (end 105.791 62.484) (width 0.5) (layer "B.Cu") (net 23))
 (segment (start 105.791 62.484) (end 100.584 62.484) (width 0.5) (layer "B.Cu") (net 23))
 (segment (start 141.605 50.165) (end 143.51 52.07) (width 0.5) (layer "B.Cu") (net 23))
 (segment (start 107.315 55.245) (end 107.315 60.96) (width 0.5) (layer "B.Cu") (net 23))
 (segment (start 113.284 53.838) (end 113.284 51.816) (width 0.5) (layer "B.Cu") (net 23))
 (segment (start 100.584 56.984) (end 105.498 52.07) (width 0.5) (layer "F.Cu") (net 16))
 (segment (start 121.92 53.34) (end 121.92 67.31) (width 0.5) (layer "F.Cu") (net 16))
 (segment (start 120.65 52.07) (end 121.92 53.34) (width 0.5) (layer "F.Cu") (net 16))
 (segment (start 121.92 67.31) (end 123.688 69.078) (width 0.5) (layer "F.Cu") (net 16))
 (segment (start 123.688 69.078) (end 138.684 69.078) (width 0.5) (layer "F.Cu") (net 16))
 (segment (start 105.498 52.07) (end 120.65 52.07) (width 0.5) (layer "F.Cu") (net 16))
 (segment (start 101.6 102.87) (end 100.584 101.854) (width 0.2) (layer "B.Cu") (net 9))
 (segment (start 138.684 86.858) (end 118.882 86.858) (width 0.2) (layer "B.Cu") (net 9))
 (segment (start 114.935 102.87) (end 101.6 102.87) (width 0.2) (layer "B.Cu") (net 9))
 (segment (start 100.584 101.854) (end 100.584 85.852) (width 0.2) (layer "B.Cu") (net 9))
 (segment (start 118.882 86.858) (end 118.11 87.63) (width 0.2) (layer "B.Cu") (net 9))
 (segment (start 118.11 87.63) (end 118.11 99.695) (width 0.2) (layer "B.Cu") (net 9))
 (segment (start 118.11 99.695) (end 114.935 102.87) (width 0.2) (layer "B.Cu") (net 9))
 (segment (start 100.584 80.352) (end 98.718 80.352) (width 0.2) (layer "B.Cu") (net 6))
 (segment (start 98.718 80.352) (end 98.425 80.645) (width 0.2) (layer "B.Cu") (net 6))
 (segment (start 136.662 94.478) (end 138.684 94.478) (width 0.2) (layer "B.Cu") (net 6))
 (segment (start 135.89 95.25) (end 136.662 94.478) (width 0.2) (layer "B.Cu") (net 6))
 (segment (start 98.425 102.235) (end 100.33 104.14) (width 0.2) (layer "B.Cu") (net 6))
 (segment (start 98.425 80.645) (end 98.425 102.235) (width 0.2) (layer "B.Cu") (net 6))
 (segment (start 100.33 104.14) (end 134.62 104.14) (width 0.2) (layer "B.Cu") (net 6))
 (segment (start 135.89 102.87) (end 135.89 95.25) (width 0.2) (layer "B.Cu") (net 6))
 (segment (start 134.62 104.14) (end 135.89 102.87) (width 0.2) (layer "B.Cu") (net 6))
 (segment (start 108.585 100.33) (end 108.585 75.565) (width 0.2) (layer "B.Cu") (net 10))
 (segment (start 116.84 99.06) (end 114.3 101.6) (width 0.2) (layer "B.Cu") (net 10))
 (segment (start 116.84 85.725) (end 116.84 99.06) (width 0.2) (layer "B.Cu") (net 10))
 (segment (start 114.3 101.6) (end 109.855 101.6) (width 0.2) (layer "B.Cu") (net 10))
 (segment (start 109.855 101.6) (end 108.585 100.33) (width 0.2) (layer "B.Cu") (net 10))
 (segment (start 118.247 84.318) (end 116.84 85.725) (width 0.2) (layer "B.Cu") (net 10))
 (segment (start 107.872 74.852) (end 100.584 74.852) (width 0.2) (layer "B.Cu") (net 10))
 (segment (start 138.684 84.318) (end 118.247 84.318) (width 0.2) (layer "B.Cu") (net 10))
 (segment (start 108.585 75.565) (end 107.872 74.852) (width 0.2) (layer "B.Cu") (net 10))
 (segment (start 79.375 93.472) (end 70.739 93.472) (width 0.5) (layer "F.Cu") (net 1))
 (segment (start 81.407 91.44) (end 79.375 93.472) (width 0.5) (layer "F.Cu") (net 1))
 (segment (start 70.739 93.472) (end 68.707 91.44) (width 0.5) (layer "F.Cu") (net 1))
 (segment (start 86.36 86.487) (end 81.407 91.44) (width 0.5) (layer "B.Cu") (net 1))
 (segment (start 86.36 65.405) (end 86.36 86.487) (width 0.5) (layer "B.Cu") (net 1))
 (segment (start 68.707 91.44) (end 68.707 84.836) (width 0.5) (layer "B.Cu") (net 1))
 (segment (start 83.439 62.484) (end 86.36 65.405) (width 0.5) (layer "B.Cu") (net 1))
 (segment (start 83.439 80.352) (end 78.867 84.924) (width 0.2) (layer "B.Cu") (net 42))
 (segment (start 78.867 84.924) (end 78.867 91.44) (width 0.2) (layer "B.Cu") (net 42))
 (segment (start 71.247 91.44) (end 76.835 85.852) (width 0.2) (layer "F.Cu") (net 43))
 (segment (start 76.835 85.852) (end 83.439 85.852) (width 0.2) (layer "F.Cu") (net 43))
 (segment (start 144.145 81.28) (end 143.647 81.778) (width 0.2) (layer "F.Cu") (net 11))
 (segment (start 144.78 72.871) (end 144.145 73.506) (width 0.2) (layer "F.Cu") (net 11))
 (segment (start 148.617 72.871) (end 144.78 72.871) (width 0.2) (layer "F.Cu") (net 11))
 (segment (start 143.647 81.778) (end 138.684 81.778) (width 0.2) (layer "F.Cu") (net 11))
 (segment (start 144.145 73.506) (end 144.145 81.28) (width 0.2) (layer "F.Cu") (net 11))
 (segment (start 153.67 92.71) (end 152.4 91.44) (width 0.2) (layer "F.Cu") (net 18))
 (segment (start 152.4 71.12) (end 145.278 63.998) (width 0.2) (layer "F.Cu") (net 18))
 (segment (start 174.498 93.853) (end 173.355 92.71) (width 0.2) (layer "F.Cu") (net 18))
 (segment (start 145.278 63.998) (end 138.684 63.998) (width 0.2) (layer "F.Cu") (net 18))
 (segment (start 152.4 91.44) (end 152.4 71.12) (width 0.2) (layer "F.Cu") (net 18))
 (segment (start 173.355 92.71) (end 153.67 92.71) (width 0.2) (layer "F.Cu") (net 18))
 (segment (start 174.498 102.87) (end 174.498 93.853) (width 0.2) (layer "F.Cu") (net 18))
 (segment (start 130.81 64.77) (end 129.042 66.538) (width 0.5) (layer "B.Cu") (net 28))
 (segment (start 171.958 95.758) (end 170.815 94.615) (width 0.5) (layer "B.Cu") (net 28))
 (segment (start 141.605 93.345) (end 141.605 52.705) (width 0.5) (layer "B.Cu") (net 28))
 (segment (start 130.81 52.705) (end 130.81 64.77) (width 0.5) (layer "B.Cu") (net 28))
 (segment (start 140.335 51.435) (end 132.08 51.435) (width 0.5) (layer "B.Cu") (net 28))
 (segment (start 142.875 94.615) (end 141.605 93.345) (width 0.5) (layer "B.Cu") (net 28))
 (segment (start 129.042 66.538) (end 113.284 66.538) (width 0.5) (layer "B.Cu") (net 28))
 (segment (start 170.815 94.615) (end 142.875 94.615) (width 0.5) (layer "B.Cu") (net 28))
 (segment (start 171.958 102.87) (end 171.958 95.758) (width 0.5) (layer "B.Cu") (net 28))
 (segment (start 132.08 51.435) (end 130.81 52.705) (width 0.5) (layer "B.Cu") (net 28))
 (segment (start 141.605 52.705) (end 140.335 51.435) (width 0.5) (layer "B.Cu") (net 28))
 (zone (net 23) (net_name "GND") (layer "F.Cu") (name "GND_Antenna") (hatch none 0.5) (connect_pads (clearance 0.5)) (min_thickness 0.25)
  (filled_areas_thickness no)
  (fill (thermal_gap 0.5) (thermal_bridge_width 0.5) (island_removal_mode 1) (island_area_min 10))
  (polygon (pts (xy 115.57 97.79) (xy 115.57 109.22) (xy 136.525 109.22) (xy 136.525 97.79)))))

